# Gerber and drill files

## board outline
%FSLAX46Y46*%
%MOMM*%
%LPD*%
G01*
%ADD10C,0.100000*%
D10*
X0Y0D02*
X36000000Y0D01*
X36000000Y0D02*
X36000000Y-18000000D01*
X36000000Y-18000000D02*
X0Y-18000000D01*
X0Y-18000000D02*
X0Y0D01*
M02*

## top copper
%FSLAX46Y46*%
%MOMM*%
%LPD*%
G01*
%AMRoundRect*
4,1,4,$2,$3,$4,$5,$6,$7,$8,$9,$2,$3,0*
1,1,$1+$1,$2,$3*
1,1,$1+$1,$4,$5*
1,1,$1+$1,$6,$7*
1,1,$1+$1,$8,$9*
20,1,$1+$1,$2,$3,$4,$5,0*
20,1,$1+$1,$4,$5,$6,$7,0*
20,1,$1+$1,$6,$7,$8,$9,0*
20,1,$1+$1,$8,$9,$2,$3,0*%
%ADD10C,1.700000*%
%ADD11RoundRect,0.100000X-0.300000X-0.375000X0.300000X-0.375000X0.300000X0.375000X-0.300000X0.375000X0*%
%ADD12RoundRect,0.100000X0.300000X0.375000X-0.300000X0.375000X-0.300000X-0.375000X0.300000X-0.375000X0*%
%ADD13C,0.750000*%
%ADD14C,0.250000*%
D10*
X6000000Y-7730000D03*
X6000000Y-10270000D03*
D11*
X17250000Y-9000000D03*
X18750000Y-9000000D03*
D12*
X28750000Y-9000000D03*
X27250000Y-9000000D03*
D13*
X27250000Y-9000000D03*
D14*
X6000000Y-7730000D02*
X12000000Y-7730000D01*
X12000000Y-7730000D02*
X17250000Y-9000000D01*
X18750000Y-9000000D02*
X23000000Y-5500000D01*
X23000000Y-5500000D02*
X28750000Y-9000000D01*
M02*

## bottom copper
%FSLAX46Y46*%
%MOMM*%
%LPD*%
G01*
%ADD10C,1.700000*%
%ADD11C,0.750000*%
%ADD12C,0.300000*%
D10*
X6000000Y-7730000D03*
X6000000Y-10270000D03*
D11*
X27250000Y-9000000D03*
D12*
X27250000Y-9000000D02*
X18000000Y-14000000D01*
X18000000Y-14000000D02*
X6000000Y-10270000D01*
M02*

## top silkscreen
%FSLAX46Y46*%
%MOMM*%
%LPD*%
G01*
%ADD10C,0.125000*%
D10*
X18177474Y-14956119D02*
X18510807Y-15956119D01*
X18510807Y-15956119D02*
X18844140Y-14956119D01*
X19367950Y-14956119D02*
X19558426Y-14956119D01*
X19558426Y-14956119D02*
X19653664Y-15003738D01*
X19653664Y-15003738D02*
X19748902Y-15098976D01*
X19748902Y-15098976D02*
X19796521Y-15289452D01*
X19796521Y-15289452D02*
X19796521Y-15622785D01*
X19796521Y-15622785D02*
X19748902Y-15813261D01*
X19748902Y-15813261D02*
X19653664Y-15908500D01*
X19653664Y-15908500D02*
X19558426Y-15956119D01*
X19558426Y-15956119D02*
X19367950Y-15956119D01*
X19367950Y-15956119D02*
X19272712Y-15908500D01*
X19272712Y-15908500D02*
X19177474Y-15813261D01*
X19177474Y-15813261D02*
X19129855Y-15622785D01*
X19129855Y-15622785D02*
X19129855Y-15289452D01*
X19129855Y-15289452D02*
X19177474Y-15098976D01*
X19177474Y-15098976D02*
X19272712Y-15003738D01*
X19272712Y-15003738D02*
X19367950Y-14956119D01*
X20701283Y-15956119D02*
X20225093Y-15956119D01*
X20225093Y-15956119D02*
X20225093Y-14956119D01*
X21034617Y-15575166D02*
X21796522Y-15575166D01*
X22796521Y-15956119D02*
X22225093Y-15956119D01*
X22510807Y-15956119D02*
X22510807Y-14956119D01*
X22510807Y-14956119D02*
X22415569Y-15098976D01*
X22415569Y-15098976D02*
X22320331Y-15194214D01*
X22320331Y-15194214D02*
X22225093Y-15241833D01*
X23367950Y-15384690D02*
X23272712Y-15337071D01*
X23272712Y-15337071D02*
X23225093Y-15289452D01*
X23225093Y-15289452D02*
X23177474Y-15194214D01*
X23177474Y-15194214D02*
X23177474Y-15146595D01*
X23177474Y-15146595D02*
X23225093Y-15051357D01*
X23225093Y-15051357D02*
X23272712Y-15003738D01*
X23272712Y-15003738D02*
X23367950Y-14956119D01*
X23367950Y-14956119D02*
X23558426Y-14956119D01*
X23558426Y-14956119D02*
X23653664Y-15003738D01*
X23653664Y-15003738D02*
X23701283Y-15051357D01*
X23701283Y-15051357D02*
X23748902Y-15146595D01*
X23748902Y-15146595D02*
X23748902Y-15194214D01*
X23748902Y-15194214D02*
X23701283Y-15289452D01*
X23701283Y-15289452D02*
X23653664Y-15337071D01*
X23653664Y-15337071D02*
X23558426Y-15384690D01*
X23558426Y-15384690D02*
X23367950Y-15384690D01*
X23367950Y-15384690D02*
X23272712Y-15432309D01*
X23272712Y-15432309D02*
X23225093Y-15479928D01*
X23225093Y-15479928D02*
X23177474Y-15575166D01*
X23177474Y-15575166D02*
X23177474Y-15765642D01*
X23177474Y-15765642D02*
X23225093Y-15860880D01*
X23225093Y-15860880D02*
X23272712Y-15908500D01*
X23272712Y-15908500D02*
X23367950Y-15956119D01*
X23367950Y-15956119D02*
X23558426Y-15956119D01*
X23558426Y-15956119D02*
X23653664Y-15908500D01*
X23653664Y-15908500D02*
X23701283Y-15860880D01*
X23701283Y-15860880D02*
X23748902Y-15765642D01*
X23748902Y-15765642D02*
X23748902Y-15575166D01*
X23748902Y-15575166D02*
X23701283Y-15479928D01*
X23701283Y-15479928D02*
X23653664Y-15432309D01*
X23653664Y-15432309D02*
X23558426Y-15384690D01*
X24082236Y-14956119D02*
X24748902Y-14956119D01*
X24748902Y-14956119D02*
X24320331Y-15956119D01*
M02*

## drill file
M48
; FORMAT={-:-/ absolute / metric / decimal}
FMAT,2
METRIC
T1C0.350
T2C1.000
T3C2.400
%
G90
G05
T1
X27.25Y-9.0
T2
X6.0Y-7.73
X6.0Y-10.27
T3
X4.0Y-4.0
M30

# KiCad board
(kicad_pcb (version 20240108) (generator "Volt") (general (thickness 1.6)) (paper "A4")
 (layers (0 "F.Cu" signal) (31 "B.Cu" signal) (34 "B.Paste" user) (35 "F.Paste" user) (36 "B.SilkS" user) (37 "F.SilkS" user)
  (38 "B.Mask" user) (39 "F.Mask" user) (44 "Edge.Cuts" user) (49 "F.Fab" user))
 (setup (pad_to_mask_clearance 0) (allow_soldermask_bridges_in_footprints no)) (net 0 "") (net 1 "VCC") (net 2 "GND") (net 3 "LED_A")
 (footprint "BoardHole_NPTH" (layer "F.Cu") (at 4 4)
  (pad "" np_thru_hole circle (at 0 0) (size 2.4 2.4) (drill 2.4) (layers "*.Cu" "*.Mask")))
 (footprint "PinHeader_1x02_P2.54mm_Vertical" (layer "F.Cu") (at 6 9)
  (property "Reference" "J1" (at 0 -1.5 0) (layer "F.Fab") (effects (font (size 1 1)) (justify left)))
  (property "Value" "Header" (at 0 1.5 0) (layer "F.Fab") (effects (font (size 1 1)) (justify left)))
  (pad "1" thru_hole circle (at 0 -1.27) (size 1.7 1.7) (drill 1) (layers "*.Cu" "*.Mask") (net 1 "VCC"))
  (pad "2" thru_hole circle (at 0 1.27) (size 1.7 1.7) (drill 1) (layers "*.Cu" "*.Mask") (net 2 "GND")))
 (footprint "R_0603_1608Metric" (layer "F.Cu") (at 18 9)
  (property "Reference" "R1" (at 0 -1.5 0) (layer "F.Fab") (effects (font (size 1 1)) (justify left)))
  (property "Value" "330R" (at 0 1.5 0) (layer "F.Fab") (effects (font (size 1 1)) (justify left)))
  (pad "1" smd roundrect (at -0.75 0) (size 0.8 0.95) (layers "F.Cu" "F.Paste" "F.Mask") (roundrect_rratio 0.125) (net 1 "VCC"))
  (pad "2" smd roundrect (at 0.75 0) (size 0.8 0.95) (layers "F.Cu" "F.Paste" "F.Mask") (roundrect_rratio 0.125) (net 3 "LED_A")))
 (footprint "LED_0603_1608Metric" (layer "F.Cu") (at 28 9 180)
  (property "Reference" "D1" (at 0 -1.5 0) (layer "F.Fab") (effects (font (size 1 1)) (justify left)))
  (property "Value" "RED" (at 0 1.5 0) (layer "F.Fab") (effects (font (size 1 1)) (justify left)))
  (pad "1" smd roundrect (at -0.75 0 180) (size 0.8 0.95) (layers "F.Cu" "F.Paste" "F.Mask") (roundrect_rratio 0.125) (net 3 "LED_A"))
  (pad "2" smd roundrect (at 0.75 0 180) (size 0.8 0.95) (layers "F.Cu" "F.Paste" "F.Mask") (roundrect_rratio 0.125) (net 2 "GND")))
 (segment (start 6 7.73) (end 12 7.73) (width 0.25) (layer "F.Cu") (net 1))
 (segment (start 12 7.73) (end 17.25 9) (width 0.25) (layer "F.Cu") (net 1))
 (segment (start 18.75 9) (end 23 5.5) (width 0.25) (layer "F.Cu") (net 3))
 (segment (start 23 5.5) (end 28.75 9) (width 0.25) (layer "F.Cu") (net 3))
 (segment (start 27.25 9) (end 18 14) (width 0.3) (layer "B.Cu") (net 2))
 (segment (start 18 14) (end 6 10.27) (width 0.3) (layer "B.Cu") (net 2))
 (via (at 27.25 9) (size 0.75) (drill 0.35) (layers "F.Cu" "B.Cu") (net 2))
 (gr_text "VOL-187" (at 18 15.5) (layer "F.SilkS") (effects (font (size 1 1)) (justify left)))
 (gr_line (start 0 0) (end 36 0) (stroke (width 0.1) (type default)) (layer "Edge.Cuts"))
 (gr_line (start 36 0) (end 36 18) (stroke (width 0.1) (type default)) (layer "Edge.Cuts"))
 (gr_line (start 36 18) (end 0 18) (stroke (width 0.1) (type default)) (layer "Edge.Cuts"))
 (gr_line (start 0 18) (end 0 0) (stroke (width 0.1) (type default)) (layer "Edge.Cuts")))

